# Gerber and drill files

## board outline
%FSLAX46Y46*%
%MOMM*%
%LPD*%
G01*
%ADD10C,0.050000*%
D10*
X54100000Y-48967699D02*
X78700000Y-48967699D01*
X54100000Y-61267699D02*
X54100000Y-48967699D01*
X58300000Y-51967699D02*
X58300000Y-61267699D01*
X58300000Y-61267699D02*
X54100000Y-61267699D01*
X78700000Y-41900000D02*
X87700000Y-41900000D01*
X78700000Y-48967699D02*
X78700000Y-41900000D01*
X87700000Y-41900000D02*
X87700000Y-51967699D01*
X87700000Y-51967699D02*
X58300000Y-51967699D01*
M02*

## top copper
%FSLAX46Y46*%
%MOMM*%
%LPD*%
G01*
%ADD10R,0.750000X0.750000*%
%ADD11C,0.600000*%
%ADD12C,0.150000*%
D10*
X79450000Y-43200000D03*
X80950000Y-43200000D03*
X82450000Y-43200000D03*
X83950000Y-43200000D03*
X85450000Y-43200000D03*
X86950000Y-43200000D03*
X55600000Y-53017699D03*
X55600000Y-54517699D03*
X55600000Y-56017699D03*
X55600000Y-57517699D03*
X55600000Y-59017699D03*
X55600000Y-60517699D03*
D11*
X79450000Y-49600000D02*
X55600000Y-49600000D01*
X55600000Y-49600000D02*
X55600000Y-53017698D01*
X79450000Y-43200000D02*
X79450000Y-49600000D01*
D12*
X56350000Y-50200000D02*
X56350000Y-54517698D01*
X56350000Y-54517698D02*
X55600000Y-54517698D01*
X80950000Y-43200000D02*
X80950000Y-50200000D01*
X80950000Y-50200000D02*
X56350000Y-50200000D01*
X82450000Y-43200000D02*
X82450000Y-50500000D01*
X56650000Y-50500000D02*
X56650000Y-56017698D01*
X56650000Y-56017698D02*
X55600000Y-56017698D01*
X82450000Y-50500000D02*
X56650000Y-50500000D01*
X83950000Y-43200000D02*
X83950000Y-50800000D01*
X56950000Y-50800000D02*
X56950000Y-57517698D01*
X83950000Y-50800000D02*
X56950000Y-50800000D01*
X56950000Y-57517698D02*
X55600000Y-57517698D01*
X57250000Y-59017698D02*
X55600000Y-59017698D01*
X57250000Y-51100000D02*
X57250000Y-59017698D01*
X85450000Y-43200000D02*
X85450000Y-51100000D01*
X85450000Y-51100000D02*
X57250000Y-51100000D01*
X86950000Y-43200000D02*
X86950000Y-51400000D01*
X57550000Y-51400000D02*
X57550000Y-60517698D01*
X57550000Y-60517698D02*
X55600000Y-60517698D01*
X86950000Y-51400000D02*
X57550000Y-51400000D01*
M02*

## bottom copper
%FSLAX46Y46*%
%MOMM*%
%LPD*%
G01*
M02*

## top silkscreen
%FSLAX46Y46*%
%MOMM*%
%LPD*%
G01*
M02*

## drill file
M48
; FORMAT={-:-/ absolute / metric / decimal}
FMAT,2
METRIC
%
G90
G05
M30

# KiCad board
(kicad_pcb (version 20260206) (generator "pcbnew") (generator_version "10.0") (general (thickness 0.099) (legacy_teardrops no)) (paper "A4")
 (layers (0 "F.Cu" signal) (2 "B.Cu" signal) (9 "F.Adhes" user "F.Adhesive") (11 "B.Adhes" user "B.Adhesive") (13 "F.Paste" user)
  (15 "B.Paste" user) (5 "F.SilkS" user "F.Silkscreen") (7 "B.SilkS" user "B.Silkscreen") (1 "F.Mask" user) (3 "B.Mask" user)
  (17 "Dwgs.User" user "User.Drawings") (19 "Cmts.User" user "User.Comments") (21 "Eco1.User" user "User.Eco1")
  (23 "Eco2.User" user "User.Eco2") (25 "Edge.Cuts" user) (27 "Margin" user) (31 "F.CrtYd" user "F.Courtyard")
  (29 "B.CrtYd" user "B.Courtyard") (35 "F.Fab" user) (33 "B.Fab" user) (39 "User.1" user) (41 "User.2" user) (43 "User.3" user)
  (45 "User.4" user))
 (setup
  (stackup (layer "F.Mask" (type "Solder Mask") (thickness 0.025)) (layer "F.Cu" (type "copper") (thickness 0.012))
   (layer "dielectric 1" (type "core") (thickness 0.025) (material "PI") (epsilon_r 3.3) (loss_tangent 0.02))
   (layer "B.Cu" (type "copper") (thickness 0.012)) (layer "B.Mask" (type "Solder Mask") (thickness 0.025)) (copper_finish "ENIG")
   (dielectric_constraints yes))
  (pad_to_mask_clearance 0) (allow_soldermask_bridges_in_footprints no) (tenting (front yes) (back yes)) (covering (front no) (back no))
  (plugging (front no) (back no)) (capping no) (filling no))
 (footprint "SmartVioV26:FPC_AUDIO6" (layer "F.Cu") (at 0 0)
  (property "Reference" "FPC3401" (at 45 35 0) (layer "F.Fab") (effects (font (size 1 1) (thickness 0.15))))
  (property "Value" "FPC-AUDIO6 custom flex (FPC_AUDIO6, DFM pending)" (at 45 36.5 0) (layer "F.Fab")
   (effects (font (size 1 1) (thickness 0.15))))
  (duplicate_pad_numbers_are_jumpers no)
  (pad "S1" smd rect (at 79.45 43.2) (size 0.75 0.75) (layers "F.Cu" "F.Mask") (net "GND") (solder_mask_margin 0.1))
  (pad "S2" smd rect (at 80.95 43.2) (size 0.75 0.75) (layers "F.Cu" "F.Mask") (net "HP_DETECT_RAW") (solder_mask_margin 0.1))
  (pad "S3" smd rect (at 82.45 43.2) (size 0.75 0.75) (layers "F.Cu" "F.Mask") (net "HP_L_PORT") (solder_mask_margin 0.1))
  (pad "S4" smd rect (at 83.95 43.2) (size 0.75 0.75) (layers "F.Cu" "F.Mask") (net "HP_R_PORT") (solder_mask_margin 0.1))
  (pad "S5" smd rect (at 85.45 43.2) (size 0.75 0.75) (layers "F.Cu" "F.Mask") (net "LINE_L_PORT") (solder_mask_margin 0.1))
  (pad "S6" smd rect (at 86.95 43.2) (size 0.75 0.75) (layers "F.Cu" "F.Mask") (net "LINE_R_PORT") (solder_mask_margin 0.1))
  (pad "T1" smd rect (at 55.6 53.017699) (size 0.75 0.75) (layers "F.Cu" "F.Mask") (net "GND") (solder_mask_margin 0.1))
  (pad "T2" smd rect (at 55.6 54.517699) (size 0.75 0.75) (layers "F.Cu" "F.Mask") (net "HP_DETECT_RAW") (solder_mask_margin 0.1))
  (pad "T3" smd rect (at 55.6 56.017699) (size 0.75 0.75) (layers "F.Cu" "F.Mask") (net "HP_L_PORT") (solder_mask_margin 0.1))
  (pad "T4" smd rect (at 55.6 57.517699) (size 0.75 0.75) (layers "F.Cu" "F.Mask") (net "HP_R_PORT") (solder_mask_margin 0.1))
  (pad "T5" smd rect (at 55.6 59.017699) (size 0.75 0.75) (layers "F.Cu" "F.Mask") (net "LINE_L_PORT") (solder_mask_margin 0.1))
  (pad "T6" smd rect (at 55.6 60.517699) (size 0.75 0.75) (layers "F.Cu" "F.Mask") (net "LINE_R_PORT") (solder_mask_margin 0.1)))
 (gr_line (start 54.1 48.967699) (end 78.7 48.967699) (stroke (width 0.05) (type default)) (layer "Edge.Cuts"))
 (gr_line (start 54.1 61.267699) (end 54.1 48.967699) (stroke (width 0.05) (type default)) (layer "Edge.Cuts"))
 (gr_line (start 58.3 51.967699) (end 58.3 61.267699) (stroke (width 0.05) (type default)) (layer "Edge.Cuts"))
 (gr_line (start 58.3 61.267699) (end 54.1 61.267699) (stroke (width 0.05) (type default)) (layer "Edge.Cuts"))
 (gr_line (start 78.7 41.9) (end 87.7 41.9) (stroke (width 0.05) (type default)) (layer "Edge.Cuts"))
 (gr_line (start 78.7 48.967699) (end 78.7 41.9) (stroke (width 0.05) (type default)) (layer "Edge.Cuts"))
 (gr_line (start 87.7 41.9) (end 87.7 51.967699) (stroke (width 0.05) (type default)) (layer "Edge.Cuts"))
 (gr_line (start 87.7 51.967699) (end 58.3 51.967699) (stroke (width 0.05) (type default)) (layer "Edge.Cuts"))
 (segment (start 79.45 49.6) (end 55.6 49.6) (width 0.6) (layer "F.Cu") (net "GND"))
 (segment (start 55.6 49.6) (end 55.6 53.017698) (width 0.6) (layer "F.Cu") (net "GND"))
 (segment (start 79.45 43.2) (end 79.45 49.6) (width 0.6) (layer "F.Cu") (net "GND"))
 (segment (start 56.35 50.2) (end 56.35 54.517698) (width 0.15) (layer "F.Cu") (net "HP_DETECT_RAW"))
 (segment (start 56.35 54.517698) (end 55.6 54.517698) (width 0.15) (layer "F.Cu") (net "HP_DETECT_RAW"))
 (segment (start 80.95 43.2) (end 80.95 50.2) (width 0.15) (layer "F.Cu") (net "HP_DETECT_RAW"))
 (segment (start 80.95 50.2) (end 56.35 50.2) (width 0.15) (layer "F.Cu") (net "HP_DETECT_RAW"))
 (segment (start 82.45 43.2) (end 82.45 50.5) (width 0.15) (layer "F.Cu") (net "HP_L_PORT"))
 (segment (start 56.65 50.5) (end 56.65 56.017698) (width 0.15) (layer "F.Cu") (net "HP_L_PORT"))
 (segment (start 56.65 56.017698) (end 55.6 56.017698) (width 0.15) (layer "F.Cu") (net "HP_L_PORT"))
 (segment (start 82.45 50.5) (end 56.65 50.5) (width 0.15) (layer "F.Cu") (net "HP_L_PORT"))
 (segment (start 83.95 43.2) (end 83.95 50.8) (width 0.15) (layer "F.Cu") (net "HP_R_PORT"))
 (segment (start 56.95 50.8) (end 56.95 57.517698) (width 0.15) (layer "F.Cu") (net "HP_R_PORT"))
 (segment (start 83.95 50.8) (end 56.95 50.8) (width 0.15) (layer "F.Cu") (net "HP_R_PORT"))
 (segment (start 56.95 57.517698) (end 55.6 57.517698) (width 0.15) (layer "F.Cu") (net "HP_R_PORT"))
 (segment (start 57.25 59.017698) (end 55.6 59.017698) (width 0.15) (layer "F.Cu") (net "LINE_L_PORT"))
 (segment (start 57.25 51.1) (end 57.25 59.017698) (width 0.15) (layer "F.Cu") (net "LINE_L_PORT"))
 (segment (start 85.45 43.2) (end 85.45 51.1) (width 0.15) (layer "F.Cu") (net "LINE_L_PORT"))
 (segment (start 85.45 51.1) (end 57.25 51.1) (width 0.15) (layer "F.Cu") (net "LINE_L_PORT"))
 (segment (start 86.95 43.2) (end 86.95 51.4) (width 0.15) (layer "F.Cu") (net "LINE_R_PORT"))
 (segment (start 57.55 51.4) (end 57.55 60.517698) (width 0.15) (layer "F.Cu") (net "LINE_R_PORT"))
 (segment (start 57.55 60.517698) (end 55.6 60.517698) (width 0.15) (layer "F.Cu") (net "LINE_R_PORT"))
 (segment (start 86.95 51.4) (end 57.55 51.4) (width 0.15) (layer "F.Cu") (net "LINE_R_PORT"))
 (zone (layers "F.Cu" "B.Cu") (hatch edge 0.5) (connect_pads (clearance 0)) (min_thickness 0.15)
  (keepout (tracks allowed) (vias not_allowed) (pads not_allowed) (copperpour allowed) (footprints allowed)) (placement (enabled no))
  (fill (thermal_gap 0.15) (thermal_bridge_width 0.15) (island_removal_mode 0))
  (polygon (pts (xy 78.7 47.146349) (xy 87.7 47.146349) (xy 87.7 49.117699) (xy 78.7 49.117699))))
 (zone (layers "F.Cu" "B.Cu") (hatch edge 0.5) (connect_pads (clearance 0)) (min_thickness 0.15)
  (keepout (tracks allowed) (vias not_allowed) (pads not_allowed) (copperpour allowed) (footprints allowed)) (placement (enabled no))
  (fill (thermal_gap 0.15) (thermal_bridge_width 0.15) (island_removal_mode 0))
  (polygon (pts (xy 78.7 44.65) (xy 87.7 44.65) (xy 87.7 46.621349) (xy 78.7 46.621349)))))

